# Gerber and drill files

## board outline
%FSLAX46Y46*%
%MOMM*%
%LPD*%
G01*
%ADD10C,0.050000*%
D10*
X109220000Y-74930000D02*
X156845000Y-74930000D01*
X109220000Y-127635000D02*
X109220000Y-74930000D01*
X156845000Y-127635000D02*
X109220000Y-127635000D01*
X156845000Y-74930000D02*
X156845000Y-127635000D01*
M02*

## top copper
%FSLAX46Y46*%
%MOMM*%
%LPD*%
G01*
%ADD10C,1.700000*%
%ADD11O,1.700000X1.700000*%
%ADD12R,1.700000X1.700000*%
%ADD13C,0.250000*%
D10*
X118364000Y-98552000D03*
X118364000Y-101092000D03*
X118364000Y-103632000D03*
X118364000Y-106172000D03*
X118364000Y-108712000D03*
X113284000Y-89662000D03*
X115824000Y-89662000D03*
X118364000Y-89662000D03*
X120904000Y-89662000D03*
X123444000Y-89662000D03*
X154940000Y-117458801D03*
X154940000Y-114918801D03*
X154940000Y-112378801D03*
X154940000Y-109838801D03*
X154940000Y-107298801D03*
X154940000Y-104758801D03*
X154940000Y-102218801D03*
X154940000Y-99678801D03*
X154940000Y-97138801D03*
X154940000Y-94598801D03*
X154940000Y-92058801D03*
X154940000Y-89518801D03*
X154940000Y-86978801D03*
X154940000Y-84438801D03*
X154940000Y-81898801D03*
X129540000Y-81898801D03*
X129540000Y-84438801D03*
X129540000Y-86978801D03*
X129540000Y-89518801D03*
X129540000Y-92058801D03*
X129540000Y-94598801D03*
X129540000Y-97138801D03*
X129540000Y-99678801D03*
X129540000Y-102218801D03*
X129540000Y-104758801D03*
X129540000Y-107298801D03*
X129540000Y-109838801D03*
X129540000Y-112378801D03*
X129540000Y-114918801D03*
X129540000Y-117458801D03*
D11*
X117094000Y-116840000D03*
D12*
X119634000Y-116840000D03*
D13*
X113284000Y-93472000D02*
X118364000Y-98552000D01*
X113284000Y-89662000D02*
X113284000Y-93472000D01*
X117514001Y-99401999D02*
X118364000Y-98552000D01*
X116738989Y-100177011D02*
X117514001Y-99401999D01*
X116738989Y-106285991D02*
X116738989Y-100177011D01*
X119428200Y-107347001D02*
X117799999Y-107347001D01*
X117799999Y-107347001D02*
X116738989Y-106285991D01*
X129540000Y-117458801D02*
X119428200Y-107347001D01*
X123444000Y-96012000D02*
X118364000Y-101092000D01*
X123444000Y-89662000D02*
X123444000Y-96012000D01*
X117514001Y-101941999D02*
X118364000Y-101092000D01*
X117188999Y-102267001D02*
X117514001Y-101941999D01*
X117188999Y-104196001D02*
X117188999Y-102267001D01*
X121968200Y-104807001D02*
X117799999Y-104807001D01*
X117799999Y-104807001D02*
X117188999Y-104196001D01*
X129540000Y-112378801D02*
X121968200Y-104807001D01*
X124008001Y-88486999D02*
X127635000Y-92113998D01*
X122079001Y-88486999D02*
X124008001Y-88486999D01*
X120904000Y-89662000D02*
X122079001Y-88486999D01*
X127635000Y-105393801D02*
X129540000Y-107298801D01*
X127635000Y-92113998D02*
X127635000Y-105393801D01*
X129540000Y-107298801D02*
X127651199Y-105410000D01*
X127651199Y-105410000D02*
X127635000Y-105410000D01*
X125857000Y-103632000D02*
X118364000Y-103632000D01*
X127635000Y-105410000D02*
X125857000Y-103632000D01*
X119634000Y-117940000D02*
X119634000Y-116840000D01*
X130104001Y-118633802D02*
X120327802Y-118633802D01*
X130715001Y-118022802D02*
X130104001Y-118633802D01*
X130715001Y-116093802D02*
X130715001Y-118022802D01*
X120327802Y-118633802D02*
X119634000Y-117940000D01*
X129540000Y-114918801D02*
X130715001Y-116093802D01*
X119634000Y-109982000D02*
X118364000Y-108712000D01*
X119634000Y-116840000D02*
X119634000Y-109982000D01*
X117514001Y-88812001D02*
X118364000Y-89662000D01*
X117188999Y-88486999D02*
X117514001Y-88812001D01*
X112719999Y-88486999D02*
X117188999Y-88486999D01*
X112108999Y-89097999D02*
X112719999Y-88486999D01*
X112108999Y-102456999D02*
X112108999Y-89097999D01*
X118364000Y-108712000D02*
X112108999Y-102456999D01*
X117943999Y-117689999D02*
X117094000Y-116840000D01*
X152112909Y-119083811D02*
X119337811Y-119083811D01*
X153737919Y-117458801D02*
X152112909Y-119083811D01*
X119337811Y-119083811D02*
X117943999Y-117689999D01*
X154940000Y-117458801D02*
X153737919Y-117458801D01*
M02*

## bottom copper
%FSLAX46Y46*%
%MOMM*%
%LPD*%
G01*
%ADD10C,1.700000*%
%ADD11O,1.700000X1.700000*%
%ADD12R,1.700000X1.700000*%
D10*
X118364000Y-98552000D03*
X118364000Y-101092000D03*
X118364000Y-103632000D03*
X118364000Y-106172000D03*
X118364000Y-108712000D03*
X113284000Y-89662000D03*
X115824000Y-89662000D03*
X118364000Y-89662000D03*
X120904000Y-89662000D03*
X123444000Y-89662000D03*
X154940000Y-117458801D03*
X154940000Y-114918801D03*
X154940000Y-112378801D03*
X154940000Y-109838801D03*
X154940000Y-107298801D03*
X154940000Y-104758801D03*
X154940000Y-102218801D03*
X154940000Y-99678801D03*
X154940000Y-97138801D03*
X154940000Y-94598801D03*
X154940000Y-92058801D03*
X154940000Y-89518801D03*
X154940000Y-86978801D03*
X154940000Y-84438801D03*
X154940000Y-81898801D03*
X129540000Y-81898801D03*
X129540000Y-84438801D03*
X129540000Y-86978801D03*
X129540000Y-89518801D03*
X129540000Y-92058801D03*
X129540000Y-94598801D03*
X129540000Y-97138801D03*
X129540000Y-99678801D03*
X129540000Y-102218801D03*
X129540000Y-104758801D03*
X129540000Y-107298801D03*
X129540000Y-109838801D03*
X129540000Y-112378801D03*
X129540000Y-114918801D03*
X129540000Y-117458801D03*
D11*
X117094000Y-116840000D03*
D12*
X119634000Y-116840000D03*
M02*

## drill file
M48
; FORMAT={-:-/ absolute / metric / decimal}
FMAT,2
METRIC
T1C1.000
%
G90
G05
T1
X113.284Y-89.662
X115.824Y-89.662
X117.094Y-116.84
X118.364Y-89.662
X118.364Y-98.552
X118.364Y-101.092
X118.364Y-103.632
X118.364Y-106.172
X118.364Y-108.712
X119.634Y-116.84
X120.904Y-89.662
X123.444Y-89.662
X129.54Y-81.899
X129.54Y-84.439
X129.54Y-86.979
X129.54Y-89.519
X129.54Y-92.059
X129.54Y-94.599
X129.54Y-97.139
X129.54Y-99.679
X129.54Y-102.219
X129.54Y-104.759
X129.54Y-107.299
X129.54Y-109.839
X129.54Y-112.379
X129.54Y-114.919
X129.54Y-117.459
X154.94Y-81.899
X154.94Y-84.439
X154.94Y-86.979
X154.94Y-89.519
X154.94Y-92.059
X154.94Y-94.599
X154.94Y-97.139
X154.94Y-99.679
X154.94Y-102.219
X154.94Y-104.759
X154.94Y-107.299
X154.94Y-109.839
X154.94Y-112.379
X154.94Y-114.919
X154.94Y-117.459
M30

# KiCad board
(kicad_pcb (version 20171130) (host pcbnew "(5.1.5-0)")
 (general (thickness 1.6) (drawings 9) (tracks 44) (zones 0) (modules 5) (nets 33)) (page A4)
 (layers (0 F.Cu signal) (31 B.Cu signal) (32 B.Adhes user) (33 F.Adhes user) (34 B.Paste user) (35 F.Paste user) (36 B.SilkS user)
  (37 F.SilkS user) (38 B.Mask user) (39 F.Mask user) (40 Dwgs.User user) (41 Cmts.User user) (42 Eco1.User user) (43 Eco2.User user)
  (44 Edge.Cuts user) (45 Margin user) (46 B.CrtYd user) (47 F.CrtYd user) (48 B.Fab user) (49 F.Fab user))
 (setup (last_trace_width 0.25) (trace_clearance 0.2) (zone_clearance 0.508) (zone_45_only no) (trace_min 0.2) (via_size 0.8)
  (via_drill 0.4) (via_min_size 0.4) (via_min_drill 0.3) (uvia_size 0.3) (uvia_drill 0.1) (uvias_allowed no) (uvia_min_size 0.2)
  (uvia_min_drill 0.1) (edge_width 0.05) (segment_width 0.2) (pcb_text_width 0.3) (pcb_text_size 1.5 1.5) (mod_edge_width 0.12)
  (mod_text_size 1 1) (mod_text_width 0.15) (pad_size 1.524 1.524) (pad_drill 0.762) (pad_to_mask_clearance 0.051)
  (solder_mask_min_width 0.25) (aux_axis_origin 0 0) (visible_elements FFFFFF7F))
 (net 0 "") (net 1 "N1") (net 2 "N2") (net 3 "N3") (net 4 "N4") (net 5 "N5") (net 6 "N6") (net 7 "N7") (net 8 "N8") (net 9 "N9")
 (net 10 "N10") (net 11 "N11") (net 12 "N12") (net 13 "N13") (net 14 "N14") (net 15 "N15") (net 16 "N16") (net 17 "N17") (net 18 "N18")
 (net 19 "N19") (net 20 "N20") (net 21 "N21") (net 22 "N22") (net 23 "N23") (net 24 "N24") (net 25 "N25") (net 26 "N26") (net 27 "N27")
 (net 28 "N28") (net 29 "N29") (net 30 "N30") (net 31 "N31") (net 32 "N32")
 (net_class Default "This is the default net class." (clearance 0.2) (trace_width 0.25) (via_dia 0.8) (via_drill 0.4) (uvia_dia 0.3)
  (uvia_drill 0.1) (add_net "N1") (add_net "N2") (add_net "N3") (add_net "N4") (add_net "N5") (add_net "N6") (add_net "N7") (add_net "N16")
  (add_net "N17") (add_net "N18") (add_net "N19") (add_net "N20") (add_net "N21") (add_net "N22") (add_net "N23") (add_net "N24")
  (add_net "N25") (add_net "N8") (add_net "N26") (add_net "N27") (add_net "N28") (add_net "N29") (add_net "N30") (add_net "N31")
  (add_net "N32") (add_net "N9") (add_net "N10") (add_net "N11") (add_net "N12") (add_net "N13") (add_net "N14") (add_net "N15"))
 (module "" (layer F.Cu) (at 131.445 114.935)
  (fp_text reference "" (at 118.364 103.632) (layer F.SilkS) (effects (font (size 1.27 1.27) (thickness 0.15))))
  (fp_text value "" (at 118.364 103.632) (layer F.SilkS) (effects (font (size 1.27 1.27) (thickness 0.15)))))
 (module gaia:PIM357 (layer F.Cu) (at 118.364 103.632 270)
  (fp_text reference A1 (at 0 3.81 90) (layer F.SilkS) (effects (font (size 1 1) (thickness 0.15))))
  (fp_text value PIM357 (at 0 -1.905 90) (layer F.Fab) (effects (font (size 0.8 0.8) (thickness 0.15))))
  (pad 1 thru_hole circle (at -5.08 0 270) (size 1.7 1.7) (drill 1) (layers *.Cu *.Mask) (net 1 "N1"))
  (pad 2 thru_hole circle (at -2.54 0 270) (size 1.7 1.7) (drill 1) (layers *.Cu *.Mask) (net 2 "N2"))
  (pad 3 thru_hole circle (at 0 0 270) (size 1.7 1.7) (drill 1) (layers *.Cu *.Mask) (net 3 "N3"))
  (pad 4 thru_hole circle (at 2.54 0 270) (size 1.7 1.7) (drill 1) (layers *.Cu *.Mask) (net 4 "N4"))
  (pad 5 thru_hole circle (at 5.08 0 270) (size 1.7 1.7) (drill 1) (layers *.Cu *.Mask) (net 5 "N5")))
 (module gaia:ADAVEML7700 (layer F.Cu) (at 118.364 84.074)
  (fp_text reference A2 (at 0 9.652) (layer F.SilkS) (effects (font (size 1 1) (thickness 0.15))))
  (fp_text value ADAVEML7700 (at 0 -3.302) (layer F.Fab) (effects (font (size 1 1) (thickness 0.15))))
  (pad 1 thru_hole circle (at -5.08 5.588) (size 1.7 1.7) (drill 1) (layers *.Cu *.Mask) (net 1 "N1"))
  (pad 2 thru_hole circle (at -2.54 5.588) (size 1.7 1.7) (drill 1) (layers *.Cu *.Mask) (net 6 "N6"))
  (pad 3 thru_hole circle (at 0 5.588) (size 1.7 1.7) (drill 1) (layers *.Cu *.Mask) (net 5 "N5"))
  (pad 4 thru_hole circle (at 2.54 5.588) (size 1.7 1.7) (drill 1) (layers *.Cu *.Mask) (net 3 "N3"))
  (pad 5 thru_hole circle (at 5.08 5.588) (size 1.7 1.7) (drill 1) (layers *.Cu *.Mask) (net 2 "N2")))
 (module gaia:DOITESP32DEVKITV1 (layer F.Cu) (at 142.24 99.678801)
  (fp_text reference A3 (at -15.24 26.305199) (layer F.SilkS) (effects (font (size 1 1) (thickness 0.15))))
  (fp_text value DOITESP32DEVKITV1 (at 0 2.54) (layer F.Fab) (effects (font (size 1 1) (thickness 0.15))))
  (pad 1 thru_hole circle (at 12.7 17.78 180) (size 1.7 1.7) (drill 1) (layers *.Cu *.Mask) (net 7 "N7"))
  (pad 2 thru_hole circle (at 12.7 15.24) (size 1.7 1.7) (drill 1) (layers *.Cu *.Mask) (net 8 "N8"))
  (pad 3 thru_hole circle (at 12.7 12.7) (size 1.7 1.7) (drill 1) (layers *.Cu *.Mask) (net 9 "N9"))
  (pad 4 thru_hole circle (at 12.7 10.16) (size 1.7 1.7) (drill 1) (layers *.Cu *.Mask) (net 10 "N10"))
  (pad 5 thru_hole circle (at 12.7 7.62) (size 1.7 1.7) (drill 1) (layers *.Cu *.Mask) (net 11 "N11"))
  (pad 6 thru_hole circle (at 12.7 5.08 90) (size 1.7 1.7) (drill 1) (layers *.Cu *.Mask) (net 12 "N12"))
  (pad 7 thru_hole circle (at 12.7 2.54) (size 1.7 1.7) (drill 1) (layers *.Cu *.Mask) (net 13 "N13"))
  (pad 8 thru_hole circle (at 12.7 0) (size 1.7 1.7) (drill 1) (layers *.Cu *.Mask) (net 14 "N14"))
  (pad 9 thru_hole circle (at 12.7 -2.54) (size 1.7 1.7) (drill 1) (layers *.Cu *.Mask) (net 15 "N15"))
  (pad 10 thru_hole circle (at 12.7 -5.08) (size 1.7 1.7) (drill 1) (layers *.Cu *.Mask) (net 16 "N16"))
  (pad 11 thru_hole circle (at 12.7 -7.62) (size 1.7 1.7) (drill 1) (layers *.Cu *.Mask) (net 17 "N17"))
  (pad 12 thru_hole circle (at 12.7 -10.16) (size 1.7 1.7) (drill 1) (layers *.Cu *.Mask) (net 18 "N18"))
  (pad 13 thru_hole circle (at 12.7 -12.7) (size 1.7 1.7) (drill 1) (layers *.Cu *.Mask) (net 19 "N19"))
  (pad 14 thru_hole circle (at 12.7 -15.24) (size 1.7 1.7) (drill 1) (layers *.Cu *.Mask) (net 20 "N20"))
  (pad 15 thru_hole circle (at 12.7 -17.78) (size 1.7 1.7) (drill 1) (layers *.Cu *.Mask) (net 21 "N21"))
  (pad 16 thru_hole circle (at -12.7 -17.78) (size 1.7 1.7) (drill 1) (layers *.Cu *.Mask) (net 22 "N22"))
  (pad 17 thru_hole circle (at -12.7 -15.24) (size 1.7 1.7) (drill 1) (layers *.Cu *.Mask) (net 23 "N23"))
  (pad 18 thru_hole circle (at -12.7 -12.7) (size 1.7 1.7) (drill 1) (layers *.Cu *.Mask) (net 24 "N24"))
  (pad 19 thru_hole circle (at -12.7 -10.16) (size 1.7 1.7) (drill 1) (layers *.Cu *.Mask) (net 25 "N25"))
  (pad 20 thru_hole circle (at -12.7 -7.62) (size 1.7 1.7) (drill 1) (layers *.Cu *.Mask) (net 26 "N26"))
  (pad 21 thru_hole circle (at -12.7 -5.08) (size 1.7 1.7) (drill 1) (layers *.Cu *.Mask) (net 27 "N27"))
  (pad 22 thru_hole circle (at -12.7 -2.54) (size 1.7 1.7) (drill 1) (layers *.Cu *.Mask) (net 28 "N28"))
  (pad 23 thru_hole circle (at -12.7 0) (size 1.7 1.7) (drill 1) (layers *.Cu *.Mask) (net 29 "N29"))
  (pad 24 thru_hole circle (at -12.7 2.54) (size 1.7 1.7) (drill 1) (layers *.Cu *.Mask) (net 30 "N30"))
  (pad 25 thru_hole circle (at -12.7 5.08) (size 1.7 1.7) (drill 1) (layers *.Cu *.Mask) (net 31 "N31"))
  (pad 26 thru_hole circle (at -12.7 7.62) (size 1.7 1.7) (drill 1) (layers *.Cu *.Mask) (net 3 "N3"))
  (pad 27 thru_hole circle (at -12.7 10.16) (size 1.7 1.7) (drill 1) (layers *.Cu *.Mask) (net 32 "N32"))
  (pad 28 thru_hole circle (at -12.7 12.7) (size 1.7 1.7) (drill 1) (layers *.Cu *.Mask) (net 2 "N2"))
  (pad 29 thru_hole circle (at -12.7 15.24) (size 1.7 1.7) (drill 1) (layers *.Cu *.Mask) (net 5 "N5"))
  (pad 30 thru_hole circle (at -12.7 17.78) (size 1.7 1.7) (drill 1) (layers *.Cu *.Mask) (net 1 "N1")))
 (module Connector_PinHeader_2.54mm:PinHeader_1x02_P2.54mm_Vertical (layer F.Cu) (at 119.634 116.84 270)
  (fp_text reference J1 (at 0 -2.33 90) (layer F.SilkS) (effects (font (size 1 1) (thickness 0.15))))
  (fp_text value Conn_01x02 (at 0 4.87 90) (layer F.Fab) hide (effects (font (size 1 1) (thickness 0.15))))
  (pad 2 thru_hole oval (at 0 2.54 270) (size 1.7 1.7) (drill 1) (layers *.Cu *.Mask) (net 7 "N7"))
  (pad 1 thru_hole rect (at 0 0 270) (size 1.7 1.7) (drill 1) (layers *.Cu *.Mask) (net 5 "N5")))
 (gr_line (start 109.22 74.93) (end 156.845 74.93) (layer Edge.Cuts) (width 0.05))
 (gr_line (start 109.22 127.635) (end 109.22 74.93) (layer Edge.Cuts) (width 0.05))
 (gr_line (start 156.845 127.635) (end 109.22 127.635) (layer Edge.Cuts) (width 0.05))
 (gr_line (start 156.845 74.93) (end 156.845 127.635) (layer Edge.Cuts) (width 0.05))
 (segment (start 113.284 93.472) (end 118.364 98.552) (width 0.25) (layer F.Cu) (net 1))
 (segment (start 113.284 89.662) (end 113.284 93.472) (width 0.25) (layer F.Cu) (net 1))
 (segment (start 117.514001 99.401999) (end 118.364 98.552) (width 0.25) (layer F.Cu) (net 1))
 (segment (start 116.738989 100.177011) (end 117.514001 99.401999) (width 0.25) (layer F.Cu) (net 1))
 (segment (start 116.738989 106.285991) (end 116.738989 100.177011) (width 0.25) (layer F.Cu) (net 1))
 (segment (start 119.4282 107.347001) (end 117.799999 107.347001) (width 0.25) (layer F.Cu) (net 1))
 (segment (start 117.799999 107.347001) (end 116.738989 106.285991) (width 0.25) (layer F.Cu) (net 1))
 (segment (start 129.54 117.458801) (end 119.4282 107.347001) (width 0.25) (layer F.Cu) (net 1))
 (segment (start 123.444 96.012) (end 118.364 101.092) (width 0.25) (layer F.Cu) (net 2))
 (segment (start 123.444 89.662) (end 123.444 96.012) (width 0.25) (layer F.Cu) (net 2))
 (segment (start 117.514001 101.941999) (end 118.364 101.092) (width 0.25) (layer F.Cu) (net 2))
 (segment (start 117.188999 102.267001) (end 117.514001 101.941999) (width 0.25) (layer F.Cu) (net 2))
 (segment (start 117.188999 104.196001) (end 117.188999 102.267001) (width 0.25) (layer F.Cu) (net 2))
 (segment (start 121.9682 104.807001) (end 117.799999 104.807001) (width 0.25) (layer F.Cu) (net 2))
 (segment (start 117.799999 104.807001) (end 117.188999 104.196001) (width 0.25) (layer F.Cu) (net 2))
 (segment (start 129.54 112.378801) (end 121.9682 104.807001) (width 0.25) (layer F.Cu) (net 2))
 (segment (start 124.008001 88.486999) (end 127.635 92.113998) (width 0.25) (layer F.Cu) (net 3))
 (segment (start 122.079001 88.486999) (end 124.008001 88.486999) (width 0.25) (layer F.Cu) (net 3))
 (segment (start 120.904 89.662) (end 122.079001 88.486999) (width 0.25) (layer F.Cu) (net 3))
 (segment (start 127.635 105.393801) (end 129.54 107.298801) (width 0.25) (layer F.Cu) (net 3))
 (segment (start 127.635 92.113998) (end 127.635 105.393801) (width 0.25) (layer F.Cu) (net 3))
 (segment (start 129.54 107.298801) (end 127.651199 105.41) (width 0.25) (layer F.Cu) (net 3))
 (segment (start 127.651199 105.41) (end 127.635 105.41) (width 0.25) (layer F.Cu) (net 3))
 (segment (start 125.857 103.632) (end 118.364 103.632) (width 0.25) (layer F.Cu) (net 3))
 (segment (start 127.635 105.41) (end 125.857 103.632) (width 0.25) (layer F.Cu) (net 3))
 (segment (start 119.634 117.94) (end 119.634 116.84) (width 0.25) (layer F.Cu) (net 5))
 (segment (start 130.104001 118.633802) (end 120.327802 118.633802) (width 0.25) (layer F.Cu) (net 5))
 (segment (start 130.715001 118.022802) (end 130.104001 118.633802) (width 0.25) (layer F.Cu) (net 5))
 (segment (start 130.715001 116.093802) (end 130.715001 118.022802) (width 0.25) (layer F.Cu) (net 5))
 (segment (start 120.327802 118.633802) (end 119.634 117.94) (width 0.25) (layer F.Cu) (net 5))
 (segment (start 129.54 114.918801) (end 130.715001 116.093802) (width 0.25) (layer F.Cu) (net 5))
 (segment (start 119.634 109.982) (end 118.364 108.712) (width 0.25) (layer F.Cu) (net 5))
 (segment (start 119.634 116.84) (end 119.634 109.982) (width 0.25) (layer F.Cu) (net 5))
 (segment (start 117.514001 88.812001) (end 118.364 89.662) (width 0.25) (layer F.Cu) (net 5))
 (segment (start 117.188999 88.486999) (end 117.514001 88.812001) (width 0.25) (layer F.Cu) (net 5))
 (segment (start 112.719999 88.486999) (end 117.188999 88.486999) (width 0.25) (layer F.Cu) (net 5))
 (segment (start 112.108999 89.097999) (end 112.719999 88.486999) (width 0.25) (layer F.Cu) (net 5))
 (segment (start 112.108999 102.456999) (end 112.108999 89.097999) (width 0.25) (layer F.Cu) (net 5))
 (segment (start 118.364 108.712) (end 112.108999 102.456999) (width 0.25) (layer F.Cu) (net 5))
 (segment (start 117.943999 117.689999) (end 117.094 116.84) (width 0.25) (layer F.Cu) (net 7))
 (segment (start 152.112909 119.083811) (end 119.337811 119.083811) (width 0.25) (layer F.Cu) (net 7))
 (segment (start 153.737919 117.458801) (end 152.112909 119.083811) (width 0.25) (layer F.Cu) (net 7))
 (segment (start 119.337811 119.083811) (end 117.943999 117.689999) (width 0.25) (layer F.Cu) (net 7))
 (segment (start 154.94 117.458801) (end 153.737919 117.458801) (width 0.25) (layer F.Cu) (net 7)))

